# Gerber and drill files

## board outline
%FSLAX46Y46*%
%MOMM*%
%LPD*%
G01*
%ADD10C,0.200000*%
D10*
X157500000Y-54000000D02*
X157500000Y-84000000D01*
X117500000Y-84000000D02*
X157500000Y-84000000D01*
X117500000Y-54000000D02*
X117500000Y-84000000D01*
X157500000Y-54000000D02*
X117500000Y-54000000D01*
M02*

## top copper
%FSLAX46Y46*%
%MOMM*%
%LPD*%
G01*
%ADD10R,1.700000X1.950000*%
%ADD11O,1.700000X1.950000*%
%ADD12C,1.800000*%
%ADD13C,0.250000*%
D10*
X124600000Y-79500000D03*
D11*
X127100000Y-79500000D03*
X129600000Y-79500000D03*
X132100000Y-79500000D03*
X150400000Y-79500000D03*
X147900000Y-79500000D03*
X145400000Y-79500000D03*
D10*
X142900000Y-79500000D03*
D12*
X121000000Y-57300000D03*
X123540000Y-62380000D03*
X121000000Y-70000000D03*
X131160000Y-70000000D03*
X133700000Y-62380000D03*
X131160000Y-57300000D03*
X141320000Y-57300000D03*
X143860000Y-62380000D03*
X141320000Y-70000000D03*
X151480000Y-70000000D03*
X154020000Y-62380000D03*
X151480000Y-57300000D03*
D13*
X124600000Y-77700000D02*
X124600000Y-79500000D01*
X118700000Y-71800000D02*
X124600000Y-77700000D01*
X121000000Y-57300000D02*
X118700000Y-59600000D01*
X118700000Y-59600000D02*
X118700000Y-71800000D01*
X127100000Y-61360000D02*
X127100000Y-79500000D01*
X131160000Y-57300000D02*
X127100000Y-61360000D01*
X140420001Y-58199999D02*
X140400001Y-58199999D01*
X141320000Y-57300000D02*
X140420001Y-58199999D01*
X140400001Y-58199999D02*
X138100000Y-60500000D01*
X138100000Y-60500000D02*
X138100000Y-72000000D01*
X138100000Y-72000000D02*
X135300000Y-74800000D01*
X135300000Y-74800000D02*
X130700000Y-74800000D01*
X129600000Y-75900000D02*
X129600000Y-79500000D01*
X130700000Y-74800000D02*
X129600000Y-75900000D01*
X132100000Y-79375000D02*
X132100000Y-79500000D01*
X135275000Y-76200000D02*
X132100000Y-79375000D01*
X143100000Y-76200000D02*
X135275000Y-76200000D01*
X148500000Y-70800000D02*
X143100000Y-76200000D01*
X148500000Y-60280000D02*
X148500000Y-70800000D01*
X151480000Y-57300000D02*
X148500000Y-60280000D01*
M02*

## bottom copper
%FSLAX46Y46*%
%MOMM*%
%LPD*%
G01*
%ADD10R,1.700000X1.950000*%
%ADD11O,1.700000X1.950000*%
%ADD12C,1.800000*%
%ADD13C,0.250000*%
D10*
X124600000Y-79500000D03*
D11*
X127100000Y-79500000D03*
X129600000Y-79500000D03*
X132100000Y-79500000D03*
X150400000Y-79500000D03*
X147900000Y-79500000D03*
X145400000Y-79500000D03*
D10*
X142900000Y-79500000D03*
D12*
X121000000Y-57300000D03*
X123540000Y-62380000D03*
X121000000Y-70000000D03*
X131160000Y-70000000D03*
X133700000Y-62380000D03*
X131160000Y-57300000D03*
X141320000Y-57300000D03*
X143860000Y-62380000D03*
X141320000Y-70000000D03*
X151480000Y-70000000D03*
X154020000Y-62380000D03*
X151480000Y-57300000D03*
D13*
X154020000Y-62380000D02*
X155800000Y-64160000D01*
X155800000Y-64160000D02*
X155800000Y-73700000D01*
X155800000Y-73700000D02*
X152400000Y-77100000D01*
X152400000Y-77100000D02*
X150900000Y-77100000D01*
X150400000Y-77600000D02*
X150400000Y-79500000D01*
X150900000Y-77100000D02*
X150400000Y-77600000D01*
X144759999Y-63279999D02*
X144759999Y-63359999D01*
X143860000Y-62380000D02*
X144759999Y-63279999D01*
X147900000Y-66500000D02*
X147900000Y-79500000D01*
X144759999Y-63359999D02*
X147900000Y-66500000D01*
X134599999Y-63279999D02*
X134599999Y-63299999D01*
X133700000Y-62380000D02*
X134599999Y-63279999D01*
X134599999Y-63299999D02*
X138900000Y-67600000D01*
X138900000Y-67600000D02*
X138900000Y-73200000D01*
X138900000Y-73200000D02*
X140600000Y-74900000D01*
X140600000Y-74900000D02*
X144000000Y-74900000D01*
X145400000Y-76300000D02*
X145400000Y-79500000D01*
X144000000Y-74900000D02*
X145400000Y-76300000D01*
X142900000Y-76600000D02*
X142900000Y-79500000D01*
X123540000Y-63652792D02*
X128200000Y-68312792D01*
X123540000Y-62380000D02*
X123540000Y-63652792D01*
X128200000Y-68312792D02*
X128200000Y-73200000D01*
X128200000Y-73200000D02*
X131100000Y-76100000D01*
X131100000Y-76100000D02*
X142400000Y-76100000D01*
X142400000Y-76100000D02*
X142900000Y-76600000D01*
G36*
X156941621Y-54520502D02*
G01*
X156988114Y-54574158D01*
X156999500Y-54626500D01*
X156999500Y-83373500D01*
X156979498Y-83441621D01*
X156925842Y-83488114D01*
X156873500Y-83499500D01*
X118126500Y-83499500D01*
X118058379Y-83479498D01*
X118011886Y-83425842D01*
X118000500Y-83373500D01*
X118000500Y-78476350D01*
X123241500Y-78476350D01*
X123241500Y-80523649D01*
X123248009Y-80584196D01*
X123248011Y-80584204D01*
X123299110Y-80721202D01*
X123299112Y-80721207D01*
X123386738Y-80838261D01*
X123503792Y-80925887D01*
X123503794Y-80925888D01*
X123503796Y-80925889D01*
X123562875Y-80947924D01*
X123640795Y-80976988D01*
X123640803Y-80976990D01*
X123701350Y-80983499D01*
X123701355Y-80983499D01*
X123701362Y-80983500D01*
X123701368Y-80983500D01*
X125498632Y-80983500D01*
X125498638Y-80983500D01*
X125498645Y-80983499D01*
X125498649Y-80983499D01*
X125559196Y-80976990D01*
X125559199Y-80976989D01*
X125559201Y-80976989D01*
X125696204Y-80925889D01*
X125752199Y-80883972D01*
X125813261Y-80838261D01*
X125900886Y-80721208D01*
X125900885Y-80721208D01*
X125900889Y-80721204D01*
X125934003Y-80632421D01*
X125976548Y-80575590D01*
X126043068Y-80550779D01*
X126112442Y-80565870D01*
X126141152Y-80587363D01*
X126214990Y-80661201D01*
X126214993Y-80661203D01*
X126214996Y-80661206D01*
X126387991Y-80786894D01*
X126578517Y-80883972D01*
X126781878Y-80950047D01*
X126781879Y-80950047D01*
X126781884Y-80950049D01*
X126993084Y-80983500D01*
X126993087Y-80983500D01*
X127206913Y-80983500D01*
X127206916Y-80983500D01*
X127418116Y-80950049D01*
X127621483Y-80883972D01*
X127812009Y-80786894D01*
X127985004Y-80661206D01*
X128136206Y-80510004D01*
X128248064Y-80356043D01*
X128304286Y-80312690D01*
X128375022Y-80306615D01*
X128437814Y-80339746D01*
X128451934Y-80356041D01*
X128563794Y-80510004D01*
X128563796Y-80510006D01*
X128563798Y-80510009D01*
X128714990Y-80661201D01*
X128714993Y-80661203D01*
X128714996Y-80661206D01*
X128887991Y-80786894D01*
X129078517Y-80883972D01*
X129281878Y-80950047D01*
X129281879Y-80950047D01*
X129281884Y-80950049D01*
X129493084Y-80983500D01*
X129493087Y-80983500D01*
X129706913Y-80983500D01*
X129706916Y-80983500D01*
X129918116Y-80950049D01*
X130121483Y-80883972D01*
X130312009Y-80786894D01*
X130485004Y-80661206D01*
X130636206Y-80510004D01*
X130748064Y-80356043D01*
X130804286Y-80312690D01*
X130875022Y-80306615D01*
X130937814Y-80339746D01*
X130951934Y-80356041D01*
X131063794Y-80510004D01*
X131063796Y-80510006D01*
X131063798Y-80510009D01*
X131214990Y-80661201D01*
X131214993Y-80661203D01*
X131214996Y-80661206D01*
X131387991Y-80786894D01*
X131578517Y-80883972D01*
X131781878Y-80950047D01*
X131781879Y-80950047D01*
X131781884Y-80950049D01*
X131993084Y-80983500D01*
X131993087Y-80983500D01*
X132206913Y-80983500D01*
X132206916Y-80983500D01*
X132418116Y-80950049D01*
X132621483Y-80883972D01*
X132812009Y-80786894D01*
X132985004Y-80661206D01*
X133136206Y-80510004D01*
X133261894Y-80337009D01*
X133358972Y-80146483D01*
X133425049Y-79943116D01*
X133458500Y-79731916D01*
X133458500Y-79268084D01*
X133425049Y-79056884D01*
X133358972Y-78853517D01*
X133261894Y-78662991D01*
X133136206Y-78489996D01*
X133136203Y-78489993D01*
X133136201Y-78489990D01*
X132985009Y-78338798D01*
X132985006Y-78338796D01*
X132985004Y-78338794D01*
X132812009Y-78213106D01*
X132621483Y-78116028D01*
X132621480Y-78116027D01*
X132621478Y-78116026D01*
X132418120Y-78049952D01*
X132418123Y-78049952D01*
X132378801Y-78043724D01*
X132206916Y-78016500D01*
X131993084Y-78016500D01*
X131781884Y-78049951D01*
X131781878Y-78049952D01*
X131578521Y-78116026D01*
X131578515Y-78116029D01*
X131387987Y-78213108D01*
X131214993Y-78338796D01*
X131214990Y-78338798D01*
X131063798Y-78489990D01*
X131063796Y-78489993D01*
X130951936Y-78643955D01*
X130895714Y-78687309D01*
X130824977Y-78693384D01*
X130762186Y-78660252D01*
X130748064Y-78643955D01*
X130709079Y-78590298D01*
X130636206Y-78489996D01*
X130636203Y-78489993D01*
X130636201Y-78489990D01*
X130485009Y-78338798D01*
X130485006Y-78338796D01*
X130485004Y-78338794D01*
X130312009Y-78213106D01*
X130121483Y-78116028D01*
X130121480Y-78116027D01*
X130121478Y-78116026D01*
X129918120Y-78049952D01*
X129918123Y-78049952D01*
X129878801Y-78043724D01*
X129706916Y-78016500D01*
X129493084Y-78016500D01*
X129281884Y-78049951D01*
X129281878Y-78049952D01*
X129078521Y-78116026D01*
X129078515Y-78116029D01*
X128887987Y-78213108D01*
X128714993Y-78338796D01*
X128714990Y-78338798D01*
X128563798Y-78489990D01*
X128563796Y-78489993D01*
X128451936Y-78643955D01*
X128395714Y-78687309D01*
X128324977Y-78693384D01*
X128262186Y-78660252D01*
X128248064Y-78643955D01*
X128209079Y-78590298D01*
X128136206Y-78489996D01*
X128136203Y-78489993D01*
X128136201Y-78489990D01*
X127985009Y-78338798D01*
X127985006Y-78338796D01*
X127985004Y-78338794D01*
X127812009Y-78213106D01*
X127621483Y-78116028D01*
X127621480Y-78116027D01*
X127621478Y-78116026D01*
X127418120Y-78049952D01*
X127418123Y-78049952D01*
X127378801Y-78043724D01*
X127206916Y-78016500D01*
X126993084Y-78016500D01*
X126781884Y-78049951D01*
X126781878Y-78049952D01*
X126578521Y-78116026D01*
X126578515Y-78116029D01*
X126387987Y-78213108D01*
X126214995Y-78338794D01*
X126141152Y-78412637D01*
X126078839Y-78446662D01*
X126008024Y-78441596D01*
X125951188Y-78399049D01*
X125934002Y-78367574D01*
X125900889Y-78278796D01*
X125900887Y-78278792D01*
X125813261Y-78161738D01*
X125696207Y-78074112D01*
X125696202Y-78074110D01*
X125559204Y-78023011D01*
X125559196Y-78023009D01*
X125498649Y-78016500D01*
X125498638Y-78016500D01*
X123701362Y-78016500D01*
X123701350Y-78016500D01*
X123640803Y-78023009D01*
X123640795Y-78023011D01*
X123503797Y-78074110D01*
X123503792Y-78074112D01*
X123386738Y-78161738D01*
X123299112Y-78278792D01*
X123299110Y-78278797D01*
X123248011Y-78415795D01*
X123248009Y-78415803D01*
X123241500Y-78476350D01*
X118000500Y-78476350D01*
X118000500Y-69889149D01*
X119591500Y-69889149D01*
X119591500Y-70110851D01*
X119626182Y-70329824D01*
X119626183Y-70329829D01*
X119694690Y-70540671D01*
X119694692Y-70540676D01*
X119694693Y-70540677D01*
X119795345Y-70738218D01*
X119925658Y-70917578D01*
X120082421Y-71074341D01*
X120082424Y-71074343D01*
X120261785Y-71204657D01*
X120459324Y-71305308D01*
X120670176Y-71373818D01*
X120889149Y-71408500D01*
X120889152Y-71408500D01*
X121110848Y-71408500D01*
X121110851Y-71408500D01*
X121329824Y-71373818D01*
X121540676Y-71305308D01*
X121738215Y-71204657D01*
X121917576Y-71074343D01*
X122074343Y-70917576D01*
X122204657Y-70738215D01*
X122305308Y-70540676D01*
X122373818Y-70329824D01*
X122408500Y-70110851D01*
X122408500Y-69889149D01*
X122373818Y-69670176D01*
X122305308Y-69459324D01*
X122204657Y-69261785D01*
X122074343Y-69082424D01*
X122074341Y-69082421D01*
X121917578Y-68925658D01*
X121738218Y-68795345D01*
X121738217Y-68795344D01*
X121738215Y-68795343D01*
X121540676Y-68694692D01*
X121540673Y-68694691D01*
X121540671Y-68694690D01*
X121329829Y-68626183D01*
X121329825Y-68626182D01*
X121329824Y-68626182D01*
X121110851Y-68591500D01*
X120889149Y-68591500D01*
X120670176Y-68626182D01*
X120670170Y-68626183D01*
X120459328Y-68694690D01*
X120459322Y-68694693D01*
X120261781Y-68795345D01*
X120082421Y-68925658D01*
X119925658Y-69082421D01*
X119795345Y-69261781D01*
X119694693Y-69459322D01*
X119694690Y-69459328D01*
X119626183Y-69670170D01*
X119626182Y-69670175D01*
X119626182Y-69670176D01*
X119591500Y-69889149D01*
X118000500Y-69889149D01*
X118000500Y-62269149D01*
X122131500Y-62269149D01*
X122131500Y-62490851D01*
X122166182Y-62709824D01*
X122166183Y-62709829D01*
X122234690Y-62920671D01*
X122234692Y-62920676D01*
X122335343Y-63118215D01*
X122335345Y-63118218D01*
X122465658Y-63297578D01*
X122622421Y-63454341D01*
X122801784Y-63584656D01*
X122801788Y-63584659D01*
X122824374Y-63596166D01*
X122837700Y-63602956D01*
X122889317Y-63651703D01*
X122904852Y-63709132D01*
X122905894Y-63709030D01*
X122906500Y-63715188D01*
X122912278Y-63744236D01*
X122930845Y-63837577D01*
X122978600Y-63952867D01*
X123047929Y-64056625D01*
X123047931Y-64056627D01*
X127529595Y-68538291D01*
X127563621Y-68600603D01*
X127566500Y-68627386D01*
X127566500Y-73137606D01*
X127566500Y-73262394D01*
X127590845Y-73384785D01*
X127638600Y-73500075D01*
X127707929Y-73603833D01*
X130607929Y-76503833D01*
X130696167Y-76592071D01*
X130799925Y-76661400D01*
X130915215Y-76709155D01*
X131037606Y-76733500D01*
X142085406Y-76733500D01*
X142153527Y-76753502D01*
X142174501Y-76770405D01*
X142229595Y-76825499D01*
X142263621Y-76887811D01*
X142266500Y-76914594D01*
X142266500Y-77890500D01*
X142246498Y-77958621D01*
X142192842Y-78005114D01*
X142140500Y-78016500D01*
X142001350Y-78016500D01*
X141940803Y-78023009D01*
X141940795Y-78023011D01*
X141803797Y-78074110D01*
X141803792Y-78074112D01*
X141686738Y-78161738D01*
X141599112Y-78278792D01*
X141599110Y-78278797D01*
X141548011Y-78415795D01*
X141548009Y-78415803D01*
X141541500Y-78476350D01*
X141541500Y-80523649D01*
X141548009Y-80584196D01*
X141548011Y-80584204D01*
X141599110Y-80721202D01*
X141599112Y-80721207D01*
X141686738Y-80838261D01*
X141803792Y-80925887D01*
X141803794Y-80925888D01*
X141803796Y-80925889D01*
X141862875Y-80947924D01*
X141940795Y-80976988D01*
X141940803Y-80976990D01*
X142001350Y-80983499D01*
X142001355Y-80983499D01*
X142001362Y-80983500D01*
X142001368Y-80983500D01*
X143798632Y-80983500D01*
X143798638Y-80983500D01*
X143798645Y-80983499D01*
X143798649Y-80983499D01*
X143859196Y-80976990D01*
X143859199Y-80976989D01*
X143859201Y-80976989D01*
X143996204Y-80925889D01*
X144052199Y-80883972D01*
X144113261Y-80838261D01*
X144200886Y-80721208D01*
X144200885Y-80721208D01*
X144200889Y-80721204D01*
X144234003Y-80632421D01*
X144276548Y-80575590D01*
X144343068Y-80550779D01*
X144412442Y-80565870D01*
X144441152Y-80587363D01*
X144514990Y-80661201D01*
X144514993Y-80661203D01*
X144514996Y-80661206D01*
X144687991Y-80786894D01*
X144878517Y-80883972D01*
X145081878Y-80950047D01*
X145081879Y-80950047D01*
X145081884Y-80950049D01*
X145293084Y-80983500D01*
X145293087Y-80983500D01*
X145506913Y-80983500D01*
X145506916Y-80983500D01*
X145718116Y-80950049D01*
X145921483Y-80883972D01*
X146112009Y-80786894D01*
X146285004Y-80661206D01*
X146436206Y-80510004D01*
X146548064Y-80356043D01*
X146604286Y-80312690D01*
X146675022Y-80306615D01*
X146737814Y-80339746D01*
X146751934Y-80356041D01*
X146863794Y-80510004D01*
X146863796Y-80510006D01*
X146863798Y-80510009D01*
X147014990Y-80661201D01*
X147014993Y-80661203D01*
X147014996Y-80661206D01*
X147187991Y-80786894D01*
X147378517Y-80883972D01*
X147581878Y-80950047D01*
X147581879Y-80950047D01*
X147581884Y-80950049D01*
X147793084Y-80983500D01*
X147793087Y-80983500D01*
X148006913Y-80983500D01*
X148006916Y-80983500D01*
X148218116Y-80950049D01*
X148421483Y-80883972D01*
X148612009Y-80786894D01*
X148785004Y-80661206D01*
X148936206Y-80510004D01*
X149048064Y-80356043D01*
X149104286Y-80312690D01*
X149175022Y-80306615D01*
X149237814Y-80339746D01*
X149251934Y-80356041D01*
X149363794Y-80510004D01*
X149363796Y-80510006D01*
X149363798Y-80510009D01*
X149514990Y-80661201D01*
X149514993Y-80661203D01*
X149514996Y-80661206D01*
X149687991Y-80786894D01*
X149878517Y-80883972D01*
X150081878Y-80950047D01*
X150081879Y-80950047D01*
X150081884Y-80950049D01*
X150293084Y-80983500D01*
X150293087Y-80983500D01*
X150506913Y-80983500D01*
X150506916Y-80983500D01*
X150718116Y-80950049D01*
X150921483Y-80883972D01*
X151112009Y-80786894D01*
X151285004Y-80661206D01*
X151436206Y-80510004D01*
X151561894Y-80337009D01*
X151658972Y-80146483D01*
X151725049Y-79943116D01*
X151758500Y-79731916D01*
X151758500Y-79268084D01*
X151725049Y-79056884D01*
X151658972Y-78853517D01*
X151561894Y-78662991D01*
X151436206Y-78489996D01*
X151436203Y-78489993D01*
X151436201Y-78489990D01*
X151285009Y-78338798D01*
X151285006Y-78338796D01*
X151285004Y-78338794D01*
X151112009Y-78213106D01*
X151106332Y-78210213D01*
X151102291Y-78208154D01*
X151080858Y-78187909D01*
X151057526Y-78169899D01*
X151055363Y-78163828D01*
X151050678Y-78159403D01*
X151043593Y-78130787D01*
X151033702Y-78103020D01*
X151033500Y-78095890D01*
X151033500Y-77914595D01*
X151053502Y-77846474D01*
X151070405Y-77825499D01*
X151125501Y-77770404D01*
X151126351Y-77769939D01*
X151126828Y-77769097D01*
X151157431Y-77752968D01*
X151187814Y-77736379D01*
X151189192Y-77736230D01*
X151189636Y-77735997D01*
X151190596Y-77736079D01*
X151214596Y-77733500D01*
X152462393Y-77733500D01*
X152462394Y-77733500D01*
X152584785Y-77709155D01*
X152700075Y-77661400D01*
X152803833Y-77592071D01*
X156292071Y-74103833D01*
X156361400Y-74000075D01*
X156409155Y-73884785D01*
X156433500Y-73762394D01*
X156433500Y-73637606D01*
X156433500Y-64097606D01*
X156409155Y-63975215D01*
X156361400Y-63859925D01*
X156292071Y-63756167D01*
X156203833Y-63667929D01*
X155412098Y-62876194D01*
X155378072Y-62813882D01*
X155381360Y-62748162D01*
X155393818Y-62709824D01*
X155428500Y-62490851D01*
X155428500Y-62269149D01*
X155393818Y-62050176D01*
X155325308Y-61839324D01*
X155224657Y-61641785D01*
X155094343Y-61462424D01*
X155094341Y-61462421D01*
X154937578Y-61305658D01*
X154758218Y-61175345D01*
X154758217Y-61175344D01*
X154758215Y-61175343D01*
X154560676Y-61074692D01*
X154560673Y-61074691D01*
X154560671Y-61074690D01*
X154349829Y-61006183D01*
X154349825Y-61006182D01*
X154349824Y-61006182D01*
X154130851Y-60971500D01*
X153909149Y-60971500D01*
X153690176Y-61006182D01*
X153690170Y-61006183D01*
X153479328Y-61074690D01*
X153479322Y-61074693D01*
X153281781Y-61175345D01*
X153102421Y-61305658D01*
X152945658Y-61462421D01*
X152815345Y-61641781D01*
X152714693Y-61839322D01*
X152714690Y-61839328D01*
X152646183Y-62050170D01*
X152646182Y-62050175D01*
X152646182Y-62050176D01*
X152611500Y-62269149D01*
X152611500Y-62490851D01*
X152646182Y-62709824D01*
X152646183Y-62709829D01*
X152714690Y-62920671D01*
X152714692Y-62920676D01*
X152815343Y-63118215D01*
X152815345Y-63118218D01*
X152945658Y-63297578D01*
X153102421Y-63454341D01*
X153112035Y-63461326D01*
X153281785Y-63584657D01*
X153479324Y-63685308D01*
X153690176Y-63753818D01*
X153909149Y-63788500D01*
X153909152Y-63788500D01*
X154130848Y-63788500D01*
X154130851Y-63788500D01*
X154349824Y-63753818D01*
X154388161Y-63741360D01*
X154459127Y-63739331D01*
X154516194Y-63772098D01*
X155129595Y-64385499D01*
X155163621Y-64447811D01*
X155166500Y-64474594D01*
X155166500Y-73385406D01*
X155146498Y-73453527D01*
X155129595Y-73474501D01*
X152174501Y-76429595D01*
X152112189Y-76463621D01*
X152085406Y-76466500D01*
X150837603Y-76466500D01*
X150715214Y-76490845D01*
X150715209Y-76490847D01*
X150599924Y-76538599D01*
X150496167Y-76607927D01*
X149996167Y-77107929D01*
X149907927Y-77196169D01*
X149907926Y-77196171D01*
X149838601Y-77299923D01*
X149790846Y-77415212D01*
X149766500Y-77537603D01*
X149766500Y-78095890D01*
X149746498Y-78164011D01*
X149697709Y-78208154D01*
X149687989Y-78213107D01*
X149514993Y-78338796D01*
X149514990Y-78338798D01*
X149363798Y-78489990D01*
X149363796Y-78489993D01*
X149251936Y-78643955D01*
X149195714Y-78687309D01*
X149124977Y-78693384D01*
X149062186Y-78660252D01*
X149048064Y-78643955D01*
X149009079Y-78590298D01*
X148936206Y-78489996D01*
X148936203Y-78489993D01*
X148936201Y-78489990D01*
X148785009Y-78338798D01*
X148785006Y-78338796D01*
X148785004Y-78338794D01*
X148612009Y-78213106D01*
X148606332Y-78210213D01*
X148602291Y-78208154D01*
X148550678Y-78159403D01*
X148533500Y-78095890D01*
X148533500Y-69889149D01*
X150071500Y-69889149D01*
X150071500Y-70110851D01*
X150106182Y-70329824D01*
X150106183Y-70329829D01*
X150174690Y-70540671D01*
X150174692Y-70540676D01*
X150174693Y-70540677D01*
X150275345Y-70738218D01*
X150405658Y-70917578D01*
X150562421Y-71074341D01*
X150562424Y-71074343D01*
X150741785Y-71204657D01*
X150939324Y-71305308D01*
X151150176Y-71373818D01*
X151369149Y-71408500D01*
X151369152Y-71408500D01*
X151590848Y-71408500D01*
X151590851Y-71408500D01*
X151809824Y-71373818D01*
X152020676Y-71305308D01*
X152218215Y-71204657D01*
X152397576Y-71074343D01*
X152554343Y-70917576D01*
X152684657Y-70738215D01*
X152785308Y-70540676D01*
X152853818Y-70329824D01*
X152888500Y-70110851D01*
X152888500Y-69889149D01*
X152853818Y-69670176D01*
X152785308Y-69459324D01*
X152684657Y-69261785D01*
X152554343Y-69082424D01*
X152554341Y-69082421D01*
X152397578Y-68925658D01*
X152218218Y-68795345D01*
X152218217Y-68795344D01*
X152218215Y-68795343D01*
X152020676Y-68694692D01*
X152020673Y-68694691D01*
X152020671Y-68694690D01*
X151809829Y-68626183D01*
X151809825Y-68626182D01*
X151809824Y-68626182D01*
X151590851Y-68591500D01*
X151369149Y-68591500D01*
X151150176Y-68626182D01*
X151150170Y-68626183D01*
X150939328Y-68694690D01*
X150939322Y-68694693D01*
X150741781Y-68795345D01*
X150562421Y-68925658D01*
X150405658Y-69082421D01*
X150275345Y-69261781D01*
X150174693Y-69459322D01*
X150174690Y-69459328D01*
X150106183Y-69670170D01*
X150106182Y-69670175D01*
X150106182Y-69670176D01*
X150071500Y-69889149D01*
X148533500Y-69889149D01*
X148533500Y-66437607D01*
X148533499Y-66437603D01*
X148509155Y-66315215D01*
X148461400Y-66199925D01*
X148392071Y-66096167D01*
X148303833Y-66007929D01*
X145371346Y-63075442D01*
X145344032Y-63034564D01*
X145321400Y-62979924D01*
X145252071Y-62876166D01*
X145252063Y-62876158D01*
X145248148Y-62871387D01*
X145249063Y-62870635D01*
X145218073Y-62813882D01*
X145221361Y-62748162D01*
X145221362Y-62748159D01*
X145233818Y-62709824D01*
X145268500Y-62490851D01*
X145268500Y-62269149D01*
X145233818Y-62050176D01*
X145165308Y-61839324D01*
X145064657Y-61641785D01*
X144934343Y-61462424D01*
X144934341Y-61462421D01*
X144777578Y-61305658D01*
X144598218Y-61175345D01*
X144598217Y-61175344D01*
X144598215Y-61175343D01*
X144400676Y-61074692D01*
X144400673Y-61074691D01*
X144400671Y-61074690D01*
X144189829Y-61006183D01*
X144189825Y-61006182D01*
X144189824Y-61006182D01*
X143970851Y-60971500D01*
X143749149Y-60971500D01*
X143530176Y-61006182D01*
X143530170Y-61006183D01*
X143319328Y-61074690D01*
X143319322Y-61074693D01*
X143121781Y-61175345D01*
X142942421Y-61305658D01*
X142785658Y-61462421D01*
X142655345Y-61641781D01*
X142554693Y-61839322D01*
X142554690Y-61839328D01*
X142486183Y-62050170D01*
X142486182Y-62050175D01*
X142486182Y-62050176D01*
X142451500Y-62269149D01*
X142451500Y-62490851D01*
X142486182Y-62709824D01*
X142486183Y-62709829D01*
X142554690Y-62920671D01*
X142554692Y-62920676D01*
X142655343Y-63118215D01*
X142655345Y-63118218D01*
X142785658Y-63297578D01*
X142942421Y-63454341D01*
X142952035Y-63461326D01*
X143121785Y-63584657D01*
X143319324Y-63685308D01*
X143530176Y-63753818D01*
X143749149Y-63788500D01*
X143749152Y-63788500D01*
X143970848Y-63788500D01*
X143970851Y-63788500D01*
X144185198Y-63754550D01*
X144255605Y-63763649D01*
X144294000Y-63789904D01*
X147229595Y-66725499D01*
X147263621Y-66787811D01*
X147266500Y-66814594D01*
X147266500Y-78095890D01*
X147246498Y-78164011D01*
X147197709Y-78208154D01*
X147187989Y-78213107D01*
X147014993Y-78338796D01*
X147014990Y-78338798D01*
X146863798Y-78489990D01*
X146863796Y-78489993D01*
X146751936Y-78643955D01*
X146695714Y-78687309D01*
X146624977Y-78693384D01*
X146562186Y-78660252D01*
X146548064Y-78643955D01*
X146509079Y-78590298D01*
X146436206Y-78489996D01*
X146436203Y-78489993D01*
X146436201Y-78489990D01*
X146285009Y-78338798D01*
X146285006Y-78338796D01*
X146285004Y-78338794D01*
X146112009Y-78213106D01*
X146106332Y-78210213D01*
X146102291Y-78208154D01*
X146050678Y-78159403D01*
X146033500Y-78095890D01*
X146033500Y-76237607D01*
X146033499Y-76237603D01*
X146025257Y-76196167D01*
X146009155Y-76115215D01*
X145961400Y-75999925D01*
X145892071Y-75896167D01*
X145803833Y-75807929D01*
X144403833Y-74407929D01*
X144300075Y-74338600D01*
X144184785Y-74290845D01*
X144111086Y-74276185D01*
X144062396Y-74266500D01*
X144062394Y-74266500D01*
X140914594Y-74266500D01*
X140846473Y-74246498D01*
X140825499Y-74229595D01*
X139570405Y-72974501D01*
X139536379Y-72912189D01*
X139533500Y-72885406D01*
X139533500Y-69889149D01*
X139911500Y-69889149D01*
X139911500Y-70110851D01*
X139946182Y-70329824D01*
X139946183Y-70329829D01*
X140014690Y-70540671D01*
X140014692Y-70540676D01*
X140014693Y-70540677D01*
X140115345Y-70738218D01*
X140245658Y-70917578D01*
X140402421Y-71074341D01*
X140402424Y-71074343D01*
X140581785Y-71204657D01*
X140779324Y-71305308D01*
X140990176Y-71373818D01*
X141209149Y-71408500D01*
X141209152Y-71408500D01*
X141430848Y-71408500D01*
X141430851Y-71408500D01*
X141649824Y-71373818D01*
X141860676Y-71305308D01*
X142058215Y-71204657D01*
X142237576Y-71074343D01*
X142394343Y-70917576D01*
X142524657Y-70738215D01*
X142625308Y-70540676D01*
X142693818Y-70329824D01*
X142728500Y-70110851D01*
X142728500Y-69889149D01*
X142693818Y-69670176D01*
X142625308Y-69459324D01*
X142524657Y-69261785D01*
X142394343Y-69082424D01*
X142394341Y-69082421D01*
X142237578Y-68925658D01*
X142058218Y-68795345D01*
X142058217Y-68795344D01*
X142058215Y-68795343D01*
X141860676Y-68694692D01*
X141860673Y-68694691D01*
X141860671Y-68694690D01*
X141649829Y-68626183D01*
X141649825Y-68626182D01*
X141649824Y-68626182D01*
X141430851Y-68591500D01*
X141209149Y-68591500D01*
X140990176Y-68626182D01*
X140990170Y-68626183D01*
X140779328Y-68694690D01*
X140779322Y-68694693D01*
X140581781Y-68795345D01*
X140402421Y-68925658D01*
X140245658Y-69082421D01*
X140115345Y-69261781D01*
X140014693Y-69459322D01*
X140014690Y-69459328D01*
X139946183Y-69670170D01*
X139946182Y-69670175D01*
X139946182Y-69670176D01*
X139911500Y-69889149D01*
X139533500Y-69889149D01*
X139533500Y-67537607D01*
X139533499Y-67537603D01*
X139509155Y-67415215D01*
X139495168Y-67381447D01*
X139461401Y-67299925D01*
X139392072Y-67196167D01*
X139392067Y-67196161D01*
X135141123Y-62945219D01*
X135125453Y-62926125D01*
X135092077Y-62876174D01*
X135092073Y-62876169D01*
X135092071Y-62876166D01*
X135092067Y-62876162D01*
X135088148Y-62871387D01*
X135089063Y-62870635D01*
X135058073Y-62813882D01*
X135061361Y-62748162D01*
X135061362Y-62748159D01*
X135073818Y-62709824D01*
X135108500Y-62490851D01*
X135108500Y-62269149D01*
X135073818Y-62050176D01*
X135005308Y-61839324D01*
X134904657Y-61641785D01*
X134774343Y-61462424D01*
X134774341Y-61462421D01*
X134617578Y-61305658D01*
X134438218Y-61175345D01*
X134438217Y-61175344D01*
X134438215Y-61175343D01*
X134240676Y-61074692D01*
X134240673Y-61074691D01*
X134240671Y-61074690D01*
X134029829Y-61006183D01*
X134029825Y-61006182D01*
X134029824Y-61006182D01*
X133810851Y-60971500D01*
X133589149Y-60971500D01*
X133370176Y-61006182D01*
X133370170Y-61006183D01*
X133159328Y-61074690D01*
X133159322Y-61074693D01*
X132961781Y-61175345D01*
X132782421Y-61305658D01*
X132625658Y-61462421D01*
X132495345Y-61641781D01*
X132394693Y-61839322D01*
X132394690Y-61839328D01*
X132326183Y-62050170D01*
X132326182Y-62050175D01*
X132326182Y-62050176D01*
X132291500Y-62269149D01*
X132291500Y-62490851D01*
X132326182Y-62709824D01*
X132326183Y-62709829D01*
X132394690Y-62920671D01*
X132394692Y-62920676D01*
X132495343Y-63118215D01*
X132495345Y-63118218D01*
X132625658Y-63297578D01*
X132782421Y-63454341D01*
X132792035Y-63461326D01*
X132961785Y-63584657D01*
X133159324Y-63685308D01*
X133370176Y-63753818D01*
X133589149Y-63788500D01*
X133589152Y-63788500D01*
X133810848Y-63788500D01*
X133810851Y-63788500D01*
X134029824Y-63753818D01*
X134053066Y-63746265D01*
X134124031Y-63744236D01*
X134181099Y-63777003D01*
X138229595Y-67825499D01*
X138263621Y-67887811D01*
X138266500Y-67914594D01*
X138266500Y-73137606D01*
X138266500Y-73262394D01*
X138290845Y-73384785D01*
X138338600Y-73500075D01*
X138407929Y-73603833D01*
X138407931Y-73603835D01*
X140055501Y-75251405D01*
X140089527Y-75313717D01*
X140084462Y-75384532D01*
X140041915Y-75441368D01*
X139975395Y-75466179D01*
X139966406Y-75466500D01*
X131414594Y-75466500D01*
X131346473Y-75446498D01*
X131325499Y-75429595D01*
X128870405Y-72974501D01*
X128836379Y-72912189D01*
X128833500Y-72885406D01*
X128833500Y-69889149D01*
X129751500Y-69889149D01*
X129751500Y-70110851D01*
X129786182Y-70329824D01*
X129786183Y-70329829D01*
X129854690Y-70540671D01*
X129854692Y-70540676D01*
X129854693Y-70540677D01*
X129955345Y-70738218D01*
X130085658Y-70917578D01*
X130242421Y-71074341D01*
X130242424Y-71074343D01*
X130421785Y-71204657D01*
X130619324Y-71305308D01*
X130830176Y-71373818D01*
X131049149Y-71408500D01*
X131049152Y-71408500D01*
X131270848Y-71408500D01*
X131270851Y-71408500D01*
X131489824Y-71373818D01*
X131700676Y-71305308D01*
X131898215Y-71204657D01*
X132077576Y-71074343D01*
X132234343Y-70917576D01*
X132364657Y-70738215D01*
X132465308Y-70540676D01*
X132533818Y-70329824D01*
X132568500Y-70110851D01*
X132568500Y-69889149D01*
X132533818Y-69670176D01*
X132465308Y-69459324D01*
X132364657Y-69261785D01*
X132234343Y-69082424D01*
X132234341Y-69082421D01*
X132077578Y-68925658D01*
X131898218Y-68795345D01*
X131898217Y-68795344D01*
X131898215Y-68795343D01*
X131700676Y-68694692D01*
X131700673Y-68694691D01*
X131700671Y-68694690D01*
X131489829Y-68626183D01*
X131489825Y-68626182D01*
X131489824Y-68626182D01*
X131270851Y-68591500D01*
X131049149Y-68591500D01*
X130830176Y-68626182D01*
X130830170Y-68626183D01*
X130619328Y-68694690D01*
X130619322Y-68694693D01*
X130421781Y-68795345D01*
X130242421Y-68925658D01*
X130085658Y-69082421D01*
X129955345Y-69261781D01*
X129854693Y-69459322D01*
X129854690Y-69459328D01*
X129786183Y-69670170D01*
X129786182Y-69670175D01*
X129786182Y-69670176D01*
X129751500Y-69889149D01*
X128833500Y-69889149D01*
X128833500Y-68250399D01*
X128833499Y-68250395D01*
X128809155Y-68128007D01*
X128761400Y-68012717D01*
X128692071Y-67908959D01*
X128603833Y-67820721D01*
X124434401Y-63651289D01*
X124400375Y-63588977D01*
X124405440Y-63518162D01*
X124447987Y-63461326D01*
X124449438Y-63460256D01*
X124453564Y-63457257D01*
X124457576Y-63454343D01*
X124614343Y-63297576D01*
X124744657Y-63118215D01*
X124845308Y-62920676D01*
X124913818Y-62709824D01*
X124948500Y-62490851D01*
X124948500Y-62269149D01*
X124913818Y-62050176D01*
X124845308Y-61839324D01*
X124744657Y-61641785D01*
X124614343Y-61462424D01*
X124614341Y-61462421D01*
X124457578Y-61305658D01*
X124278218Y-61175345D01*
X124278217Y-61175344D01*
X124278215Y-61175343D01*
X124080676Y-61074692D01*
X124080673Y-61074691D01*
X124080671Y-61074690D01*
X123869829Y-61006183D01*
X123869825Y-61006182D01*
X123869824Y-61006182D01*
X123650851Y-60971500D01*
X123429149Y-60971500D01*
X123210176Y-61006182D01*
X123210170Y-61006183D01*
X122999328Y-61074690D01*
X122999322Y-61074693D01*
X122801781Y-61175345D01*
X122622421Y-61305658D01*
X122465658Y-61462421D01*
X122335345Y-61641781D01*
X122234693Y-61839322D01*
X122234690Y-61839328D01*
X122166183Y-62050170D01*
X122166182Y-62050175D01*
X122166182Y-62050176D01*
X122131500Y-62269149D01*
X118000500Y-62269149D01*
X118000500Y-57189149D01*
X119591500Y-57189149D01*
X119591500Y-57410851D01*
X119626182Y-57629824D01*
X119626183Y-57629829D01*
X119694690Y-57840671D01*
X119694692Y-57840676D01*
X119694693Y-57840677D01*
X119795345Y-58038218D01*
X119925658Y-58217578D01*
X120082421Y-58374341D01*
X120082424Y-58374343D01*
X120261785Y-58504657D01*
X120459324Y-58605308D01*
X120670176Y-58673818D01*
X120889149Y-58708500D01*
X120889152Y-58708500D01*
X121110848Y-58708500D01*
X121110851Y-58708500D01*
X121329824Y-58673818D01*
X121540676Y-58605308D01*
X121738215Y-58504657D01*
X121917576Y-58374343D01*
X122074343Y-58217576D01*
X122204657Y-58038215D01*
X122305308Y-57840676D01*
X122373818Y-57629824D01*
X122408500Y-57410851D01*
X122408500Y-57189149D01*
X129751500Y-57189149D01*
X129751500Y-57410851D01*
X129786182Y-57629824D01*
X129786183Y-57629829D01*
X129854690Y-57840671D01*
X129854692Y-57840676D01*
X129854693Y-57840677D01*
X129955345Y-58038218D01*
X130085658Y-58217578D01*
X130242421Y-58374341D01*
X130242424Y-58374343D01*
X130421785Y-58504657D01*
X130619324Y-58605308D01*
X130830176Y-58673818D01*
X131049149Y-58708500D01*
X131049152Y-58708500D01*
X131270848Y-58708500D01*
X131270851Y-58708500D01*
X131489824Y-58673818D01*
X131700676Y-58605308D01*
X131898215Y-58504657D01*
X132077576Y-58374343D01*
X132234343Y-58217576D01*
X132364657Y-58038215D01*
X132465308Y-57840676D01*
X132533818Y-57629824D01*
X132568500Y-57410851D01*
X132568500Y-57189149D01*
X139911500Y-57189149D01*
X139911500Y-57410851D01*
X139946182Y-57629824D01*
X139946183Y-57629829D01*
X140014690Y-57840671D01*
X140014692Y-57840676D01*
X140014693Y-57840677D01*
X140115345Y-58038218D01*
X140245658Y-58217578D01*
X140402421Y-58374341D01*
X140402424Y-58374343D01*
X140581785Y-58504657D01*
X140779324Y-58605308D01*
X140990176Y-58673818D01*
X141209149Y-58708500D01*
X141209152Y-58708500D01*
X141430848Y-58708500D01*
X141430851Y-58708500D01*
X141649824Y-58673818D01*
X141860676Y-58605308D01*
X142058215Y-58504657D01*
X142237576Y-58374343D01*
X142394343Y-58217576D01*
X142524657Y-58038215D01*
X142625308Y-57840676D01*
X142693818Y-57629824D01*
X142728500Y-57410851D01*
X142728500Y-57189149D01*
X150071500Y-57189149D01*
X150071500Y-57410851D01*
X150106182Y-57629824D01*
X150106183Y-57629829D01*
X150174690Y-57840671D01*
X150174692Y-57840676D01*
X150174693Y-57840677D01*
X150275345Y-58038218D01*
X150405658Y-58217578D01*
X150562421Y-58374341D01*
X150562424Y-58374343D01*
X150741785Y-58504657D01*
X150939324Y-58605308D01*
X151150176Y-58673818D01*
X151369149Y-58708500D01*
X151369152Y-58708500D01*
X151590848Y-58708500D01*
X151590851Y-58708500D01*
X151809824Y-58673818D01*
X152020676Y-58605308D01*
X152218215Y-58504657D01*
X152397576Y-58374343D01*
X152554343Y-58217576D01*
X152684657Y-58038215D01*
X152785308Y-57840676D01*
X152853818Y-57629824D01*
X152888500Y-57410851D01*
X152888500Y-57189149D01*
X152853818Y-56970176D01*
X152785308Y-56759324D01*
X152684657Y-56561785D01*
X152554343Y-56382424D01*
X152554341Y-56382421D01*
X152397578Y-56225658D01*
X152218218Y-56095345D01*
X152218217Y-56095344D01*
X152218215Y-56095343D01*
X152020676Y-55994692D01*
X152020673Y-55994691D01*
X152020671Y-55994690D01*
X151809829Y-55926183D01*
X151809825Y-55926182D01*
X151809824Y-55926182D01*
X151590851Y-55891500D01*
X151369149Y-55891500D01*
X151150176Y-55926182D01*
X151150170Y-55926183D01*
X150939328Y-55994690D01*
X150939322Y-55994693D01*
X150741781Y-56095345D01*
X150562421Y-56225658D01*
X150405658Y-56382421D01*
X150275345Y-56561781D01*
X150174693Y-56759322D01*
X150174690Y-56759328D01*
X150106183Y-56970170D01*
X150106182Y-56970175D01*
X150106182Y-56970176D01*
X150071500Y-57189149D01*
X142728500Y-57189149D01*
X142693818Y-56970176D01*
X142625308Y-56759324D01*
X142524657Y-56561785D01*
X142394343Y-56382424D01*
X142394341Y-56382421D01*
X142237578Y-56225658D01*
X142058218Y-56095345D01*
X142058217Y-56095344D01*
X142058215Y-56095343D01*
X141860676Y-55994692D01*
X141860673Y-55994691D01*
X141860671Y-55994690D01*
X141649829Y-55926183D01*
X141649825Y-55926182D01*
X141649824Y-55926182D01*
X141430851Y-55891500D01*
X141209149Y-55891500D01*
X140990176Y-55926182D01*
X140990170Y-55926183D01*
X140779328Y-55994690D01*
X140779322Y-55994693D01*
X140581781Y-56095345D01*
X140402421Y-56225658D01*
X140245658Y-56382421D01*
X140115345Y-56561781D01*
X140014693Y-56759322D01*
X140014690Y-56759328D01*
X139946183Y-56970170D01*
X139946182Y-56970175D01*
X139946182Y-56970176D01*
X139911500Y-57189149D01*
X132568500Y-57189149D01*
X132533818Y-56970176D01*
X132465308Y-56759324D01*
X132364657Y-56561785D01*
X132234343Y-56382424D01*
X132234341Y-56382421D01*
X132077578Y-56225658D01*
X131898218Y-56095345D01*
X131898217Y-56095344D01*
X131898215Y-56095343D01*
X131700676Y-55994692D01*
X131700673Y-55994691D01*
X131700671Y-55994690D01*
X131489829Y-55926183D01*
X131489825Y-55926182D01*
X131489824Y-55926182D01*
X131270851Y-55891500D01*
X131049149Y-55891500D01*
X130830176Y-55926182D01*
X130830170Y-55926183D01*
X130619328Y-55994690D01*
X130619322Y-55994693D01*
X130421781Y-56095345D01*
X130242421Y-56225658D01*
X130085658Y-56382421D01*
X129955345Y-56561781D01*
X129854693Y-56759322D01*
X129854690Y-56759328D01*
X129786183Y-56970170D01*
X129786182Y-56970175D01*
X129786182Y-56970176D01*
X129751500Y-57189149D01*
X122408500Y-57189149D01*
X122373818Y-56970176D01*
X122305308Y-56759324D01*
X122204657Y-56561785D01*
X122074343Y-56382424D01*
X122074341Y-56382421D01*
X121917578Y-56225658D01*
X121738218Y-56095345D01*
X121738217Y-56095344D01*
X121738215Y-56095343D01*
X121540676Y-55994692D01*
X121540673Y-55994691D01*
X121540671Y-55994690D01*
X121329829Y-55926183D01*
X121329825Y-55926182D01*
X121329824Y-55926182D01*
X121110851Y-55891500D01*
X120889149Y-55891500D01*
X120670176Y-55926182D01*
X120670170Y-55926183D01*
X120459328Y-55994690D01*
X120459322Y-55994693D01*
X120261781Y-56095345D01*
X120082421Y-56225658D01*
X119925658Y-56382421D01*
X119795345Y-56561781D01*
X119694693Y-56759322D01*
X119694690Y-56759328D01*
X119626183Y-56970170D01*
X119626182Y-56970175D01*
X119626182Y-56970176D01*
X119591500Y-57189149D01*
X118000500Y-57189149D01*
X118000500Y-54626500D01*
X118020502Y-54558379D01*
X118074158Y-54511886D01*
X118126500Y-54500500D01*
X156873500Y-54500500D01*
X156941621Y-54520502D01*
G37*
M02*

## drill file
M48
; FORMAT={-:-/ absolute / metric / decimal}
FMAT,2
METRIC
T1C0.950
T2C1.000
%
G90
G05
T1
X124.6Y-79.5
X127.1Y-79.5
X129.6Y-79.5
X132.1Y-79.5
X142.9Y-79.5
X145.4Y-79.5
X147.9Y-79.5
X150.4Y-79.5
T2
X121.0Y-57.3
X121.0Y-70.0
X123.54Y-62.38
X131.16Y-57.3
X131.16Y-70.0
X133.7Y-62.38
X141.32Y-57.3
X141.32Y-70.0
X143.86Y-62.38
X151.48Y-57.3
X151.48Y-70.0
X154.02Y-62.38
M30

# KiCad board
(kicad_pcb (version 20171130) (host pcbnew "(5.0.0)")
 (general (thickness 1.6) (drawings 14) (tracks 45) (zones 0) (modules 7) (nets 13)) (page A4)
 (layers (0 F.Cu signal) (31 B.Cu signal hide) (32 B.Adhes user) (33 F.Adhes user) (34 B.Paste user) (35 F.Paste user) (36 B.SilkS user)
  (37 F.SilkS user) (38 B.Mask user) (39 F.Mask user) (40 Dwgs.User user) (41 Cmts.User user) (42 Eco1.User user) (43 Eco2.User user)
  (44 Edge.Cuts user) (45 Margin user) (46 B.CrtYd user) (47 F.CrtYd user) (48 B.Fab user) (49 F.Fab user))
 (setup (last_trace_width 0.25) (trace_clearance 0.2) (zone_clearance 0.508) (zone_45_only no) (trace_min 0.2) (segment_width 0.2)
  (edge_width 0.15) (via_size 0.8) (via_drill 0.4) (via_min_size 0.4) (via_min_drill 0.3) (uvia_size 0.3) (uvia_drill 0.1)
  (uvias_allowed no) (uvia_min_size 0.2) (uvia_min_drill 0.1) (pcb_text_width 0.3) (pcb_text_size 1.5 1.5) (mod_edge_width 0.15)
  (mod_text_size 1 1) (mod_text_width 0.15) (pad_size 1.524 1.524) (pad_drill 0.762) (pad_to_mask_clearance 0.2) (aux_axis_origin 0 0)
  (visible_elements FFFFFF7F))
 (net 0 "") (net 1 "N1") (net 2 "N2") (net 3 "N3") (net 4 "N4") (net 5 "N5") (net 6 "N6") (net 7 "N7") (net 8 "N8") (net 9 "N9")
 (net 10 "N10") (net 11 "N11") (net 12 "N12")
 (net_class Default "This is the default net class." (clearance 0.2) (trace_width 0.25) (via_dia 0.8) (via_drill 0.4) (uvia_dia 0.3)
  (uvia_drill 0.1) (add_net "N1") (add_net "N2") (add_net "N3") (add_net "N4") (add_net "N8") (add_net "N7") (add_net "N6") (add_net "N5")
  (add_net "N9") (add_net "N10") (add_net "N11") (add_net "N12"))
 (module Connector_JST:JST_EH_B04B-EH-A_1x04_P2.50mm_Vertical (layer F.Cu) (at 124.6 79.5)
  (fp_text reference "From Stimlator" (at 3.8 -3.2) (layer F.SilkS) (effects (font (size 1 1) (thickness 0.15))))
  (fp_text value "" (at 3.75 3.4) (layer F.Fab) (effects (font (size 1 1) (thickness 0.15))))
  (pad 1 thru_hole rect (at 0 0) (size 1.7 1.95) (drill 0.95) (layers *.Cu *.Mask) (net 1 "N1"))
  (pad 2 thru_hole oval (at 2.5 0) (size 1.7 1.95) (drill 0.95) (layers *.Cu *.Mask) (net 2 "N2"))
  (pad 3 thru_hole oval (at 5 0) (size 1.7 1.95) (drill 0.95) (layers *.Cu *.Mask) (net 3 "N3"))
  (pad 4 thru_hole oval (at 7.5 0) (size 1.7 1.95) (drill 0.95) (layers *.Cu *.Mask) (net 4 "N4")))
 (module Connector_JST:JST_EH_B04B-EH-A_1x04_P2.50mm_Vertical (layer F.Cu) (at 142.9 79.5)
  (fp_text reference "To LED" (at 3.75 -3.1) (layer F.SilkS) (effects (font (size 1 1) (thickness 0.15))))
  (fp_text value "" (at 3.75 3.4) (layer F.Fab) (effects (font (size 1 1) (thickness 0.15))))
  (pad 4 thru_hole oval (at 7.5 0) (size 1.7 1.95) (drill 0.95) (layers *.Cu *.Mask) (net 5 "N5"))
  (pad 3 thru_hole oval (at 5 0) (size 1.7 1.95) (drill 0.95) (layers *.Cu *.Mask) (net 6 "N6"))
  (pad 2 thru_hole oval (at 2.5 0) (size 1.7 1.95) (drill 0.95) (layers *.Cu *.Mask) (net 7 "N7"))
  (pad 1 thru_hole rect (at 0 0) (size 1.7 1.95) (drill 0.95) (layers *.Cu *.Mask) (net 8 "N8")))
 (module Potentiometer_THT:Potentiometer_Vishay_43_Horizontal (layer F.Cu) (at 121 70 270)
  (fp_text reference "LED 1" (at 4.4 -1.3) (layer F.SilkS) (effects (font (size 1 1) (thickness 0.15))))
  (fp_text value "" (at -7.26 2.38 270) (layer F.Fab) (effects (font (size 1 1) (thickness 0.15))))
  (pad 3 thru_hole circle (at -12.7 0 270) (size 1.8 1.8) (drill 1) (layers *.Cu *.Mask) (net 1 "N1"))
  (pad 2 thru_hole circle (at -7.62 -2.54 270) (size 1.8 1.8) (drill 1) (layers *.Cu *.Mask) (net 8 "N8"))
  (pad 1 thru_hole circle (at 0 0 270) (size 1.8 1.8) (drill 1) (layers *.Cu *.Mask) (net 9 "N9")))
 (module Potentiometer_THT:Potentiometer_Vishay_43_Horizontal (layer F.Cu) (at 131.16 70 270)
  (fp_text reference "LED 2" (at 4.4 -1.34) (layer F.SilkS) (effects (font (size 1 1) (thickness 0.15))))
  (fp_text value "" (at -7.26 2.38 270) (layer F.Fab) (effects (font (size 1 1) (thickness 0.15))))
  (pad 1 thru_hole circle (at 0 0 270) (size 1.8 1.8) (drill 1) (layers *.Cu *.Mask) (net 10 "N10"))
  (pad 2 thru_hole circle (at -7.62 -2.54 270) (size 1.8 1.8) (drill 1) (layers *.Cu *.Mask) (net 7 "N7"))
  (pad 3 thru_hole circle (at -12.7 0 270) (size 1.8 1.8) (drill 1) (layers *.Cu *.Mask) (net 2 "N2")))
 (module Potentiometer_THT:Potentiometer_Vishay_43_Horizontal (layer F.Cu) (at 141.32 70 270)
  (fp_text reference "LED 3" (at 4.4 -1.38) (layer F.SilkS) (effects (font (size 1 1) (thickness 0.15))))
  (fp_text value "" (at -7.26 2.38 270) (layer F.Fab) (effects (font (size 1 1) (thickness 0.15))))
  (pad 3 thru_hole circle (at -12.7 0 270) (size 1.8 1.8) (drill 1) (layers *.Cu *.Mask) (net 3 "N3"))
  (pad 2 thru_hole circle (at -7.62 -2.54 270) (size 1.8 1.8) (drill 1) (layers *.Cu *.Mask) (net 6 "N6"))
  (pad 1 thru_hole circle (at 0 0 270) (size 1.8 1.8) (drill 1) (layers *.Cu *.Mask) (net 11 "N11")))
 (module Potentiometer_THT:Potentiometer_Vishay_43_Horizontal (layer F.Cu) (at 151.48 70 270)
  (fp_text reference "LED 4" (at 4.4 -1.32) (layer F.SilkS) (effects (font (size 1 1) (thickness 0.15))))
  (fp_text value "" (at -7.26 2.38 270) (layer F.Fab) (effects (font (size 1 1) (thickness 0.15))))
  (pad 1 thru_hole circle (at 0 0 270) (size 1.8 1.8) (drill 1) (layers *.Cu *.Mask) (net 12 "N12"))
  (pad 2 thru_hole circle (at -7.62 -2.54 270) (size 1.8 1.8) (drill 1) (layers *.Cu *.Mask) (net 5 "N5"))
  (pad 3 thru_hole circle (at -12.7 0 270) (size 1.8 1.8) (drill 1) (layers *.Cu *.Mask) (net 4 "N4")))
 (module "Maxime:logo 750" (layer B.Cu) (at 137.5 75.1 180)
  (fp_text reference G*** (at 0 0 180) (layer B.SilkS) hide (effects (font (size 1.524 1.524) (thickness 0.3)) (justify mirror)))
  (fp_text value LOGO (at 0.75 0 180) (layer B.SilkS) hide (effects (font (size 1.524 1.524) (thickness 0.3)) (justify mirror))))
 (gr_line (start 157.5 54) (end 157.5 84) (layer Edge.Cuts) (width 0.2))
 (gr_line (start 117.5 84) (end 157.5 84) (layer Edge.Cuts) (width 0.2))
 (gr_line (start 117.5 54) (end 117.5 84) (layer Edge.Cuts) (width 0.2))
 (gr_line (start 157.5 54) (end 117.5 54) (layer Edge.Cuts) (width 0.2))
 (segment (start 124.6 77.7) (end 124.6 79.5) (width 0.25) (layer F.Cu) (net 1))
 (segment (start 118.7 71.8) (end 124.6 77.7) (width 0.25) (layer F.Cu) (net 1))
 (segment (start 121 57.3) (end 118.7 59.6) (width 0.25) (layer F.Cu) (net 1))
 (segment (start 118.7 59.6) (end 118.7 71.8) (width 0.25) (layer F.Cu) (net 1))
 (segment (start 127.1 61.36) (end 127.1 79.5) (width 0.25) (layer F.Cu) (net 2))
 (segment (start 131.16 57.3) (end 127.1 61.36) (width 0.25) (layer F.Cu) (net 2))
 (segment (start 140.420001 58.199999) (end 140.400001 58.199999) (width 0.25) (layer F.Cu) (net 3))
 (segment (start 141.32 57.3) (end 140.420001 58.199999) (width 0.25) (layer F.Cu) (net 3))
 (segment (start 140.400001 58.199999) (end 138.1 60.5) (width 0.25) (layer F.Cu) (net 3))
 (segment (start 138.1 60.5) (end 138.1 72) (width 0.25) (layer F.Cu) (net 3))
 (segment (start 138.1 72) (end 135.3 74.8) (width 0.25) (layer F.Cu) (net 3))
 (segment (start 135.3 74.8) (end 130.7 74.8) (width 0.25) (layer F.Cu) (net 3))
 (segment (start 129.6 75.9) (end 129.6 79.5) (width 0.25) (layer F.Cu) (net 3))
 (segment (start 130.7 74.8) (end 129.6 75.9) (width 0.25) (layer F.Cu) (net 3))
 (segment (start 132.1 79.375) (end 132.1 79.5) (width 0.25) (layer F.Cu) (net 4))
 (segment (start 135.275 76.2) (end 132.1 79.375) (width 0.25) (layer F.Cu) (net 4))
 (segment (start 143.1 76.2) (end 135.275 76.2) (width 0.25) (layer F.Cu) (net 4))
 (segment (start 148.5 70.8) (end 143.1 76.2) (width 0.25) (layer F.Cu) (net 4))
 (segment (start 148.5 60.28) (end 148.5 70.8) (width 0.25) (layer F.Cu) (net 4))
 (segment (start 151.48 57.3) (end 148.5 60.28) (width 0.25) (layer F.Cu) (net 4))
 (segment (start 154.02 62.38) (end 155.8 64.16) (width 0.25) (layer B.Cu) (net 5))
 (segment (start 155.8 64.16) (end 155.8 73.7) (width 0.25) (layer B.Cu) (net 5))
 (segment (start 155.8 73.7) (end 152.4 77.1) (width 0.25) (layer B.Cu) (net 5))
 (segment (start 152.4 77.1) (end 150.9 77.1) (width 0.25) (layer B.Cu) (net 5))
 (segment (start 150.4 77.6) (end 150.4 79.5) (width 0.25) (layer B.Cu) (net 5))
 (segment (start 150.9 77.1) (end 150.4 77.6) (width 0.25) (layer B.Cu) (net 5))
 (segment (start 144.759999 63.279999) (end 144.759999 63.359999) (width 0.25) (layer B.Cu) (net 6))
 (segment (start 143.86 62.38) (end 144.759999 63.279999) (width 0.25) (layer B.Cu) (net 6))
 (segment (start 147.9 66.5) (end 147.9 79.5) (width 0.25) (layer B.Cu) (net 6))
 (segment (start 144.759999 63.359999) (end 147.9 66.5) (width 0.25) (layer B.Cu) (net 6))
 (segment (start 134.599999 63.279999) (end 134.599999 63.299999) (width 0.25) (layer B.Cu) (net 7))
 (segment (start 133.7 62.38) (end 134.599999 63.279999) (width 0.25) (layer B.Cu) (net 7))
 (segment (start 134.599999 63.299999) (end 138.9 67.6) (width 0.25) (layer B.Cu) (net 7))
 (segment (start 138.9 67.6) (end 138.9 73.2) (width 0.25) (layer B.Cu) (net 7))
 (segment (start 138.9 73.2) (end 140.6 74.9) (width 0.25) (layer B.Cu) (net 7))
 (segment (start 140.6 74.9) (end 144 74.9) (width 0.25) (layer B.Cu) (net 7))
 (segment (start 145.4 76.3) (end 145.4 79.5) (width 0.25) (layer B.Cu) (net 7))
 (segment (start 144 74.9) (end 145.4 76.3) (width 0.25) (layer B.Cu) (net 7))
 (segment (start 142.9 76.6) (end 142.9 79.5) (width 0.25) (layer B.Cu) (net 8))
 (segment (start 123.54 63.652792) (end 128.2 68.312792) (width 0.25) (layer B.Cu) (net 8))
 (segment (start 123.54 62.38) (end 123.54 63.652792) (width 0.25) (layer B.Cu) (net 8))
 (segment (start 128.2 68.312792) (end 128.2 73.2) (width 0.25) (layer B.Cu) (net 8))
 (segment (start 128.2 73.2) (end 131.1 76.1) (width 0.25) (layer B.Cu) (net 8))
 (segment (start 131.1 76.1) (end 142.4 76.1) (width 0.25) (layer B.Cu) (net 8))
 (segment (start 142.4 76.1) (end 142.9 76.6) (width 0.25) (layer B.Cu) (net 8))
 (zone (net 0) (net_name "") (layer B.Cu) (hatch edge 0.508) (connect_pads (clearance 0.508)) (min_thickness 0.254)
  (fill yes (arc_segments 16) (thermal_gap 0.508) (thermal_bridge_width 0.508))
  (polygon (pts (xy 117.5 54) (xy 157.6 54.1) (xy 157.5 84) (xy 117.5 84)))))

